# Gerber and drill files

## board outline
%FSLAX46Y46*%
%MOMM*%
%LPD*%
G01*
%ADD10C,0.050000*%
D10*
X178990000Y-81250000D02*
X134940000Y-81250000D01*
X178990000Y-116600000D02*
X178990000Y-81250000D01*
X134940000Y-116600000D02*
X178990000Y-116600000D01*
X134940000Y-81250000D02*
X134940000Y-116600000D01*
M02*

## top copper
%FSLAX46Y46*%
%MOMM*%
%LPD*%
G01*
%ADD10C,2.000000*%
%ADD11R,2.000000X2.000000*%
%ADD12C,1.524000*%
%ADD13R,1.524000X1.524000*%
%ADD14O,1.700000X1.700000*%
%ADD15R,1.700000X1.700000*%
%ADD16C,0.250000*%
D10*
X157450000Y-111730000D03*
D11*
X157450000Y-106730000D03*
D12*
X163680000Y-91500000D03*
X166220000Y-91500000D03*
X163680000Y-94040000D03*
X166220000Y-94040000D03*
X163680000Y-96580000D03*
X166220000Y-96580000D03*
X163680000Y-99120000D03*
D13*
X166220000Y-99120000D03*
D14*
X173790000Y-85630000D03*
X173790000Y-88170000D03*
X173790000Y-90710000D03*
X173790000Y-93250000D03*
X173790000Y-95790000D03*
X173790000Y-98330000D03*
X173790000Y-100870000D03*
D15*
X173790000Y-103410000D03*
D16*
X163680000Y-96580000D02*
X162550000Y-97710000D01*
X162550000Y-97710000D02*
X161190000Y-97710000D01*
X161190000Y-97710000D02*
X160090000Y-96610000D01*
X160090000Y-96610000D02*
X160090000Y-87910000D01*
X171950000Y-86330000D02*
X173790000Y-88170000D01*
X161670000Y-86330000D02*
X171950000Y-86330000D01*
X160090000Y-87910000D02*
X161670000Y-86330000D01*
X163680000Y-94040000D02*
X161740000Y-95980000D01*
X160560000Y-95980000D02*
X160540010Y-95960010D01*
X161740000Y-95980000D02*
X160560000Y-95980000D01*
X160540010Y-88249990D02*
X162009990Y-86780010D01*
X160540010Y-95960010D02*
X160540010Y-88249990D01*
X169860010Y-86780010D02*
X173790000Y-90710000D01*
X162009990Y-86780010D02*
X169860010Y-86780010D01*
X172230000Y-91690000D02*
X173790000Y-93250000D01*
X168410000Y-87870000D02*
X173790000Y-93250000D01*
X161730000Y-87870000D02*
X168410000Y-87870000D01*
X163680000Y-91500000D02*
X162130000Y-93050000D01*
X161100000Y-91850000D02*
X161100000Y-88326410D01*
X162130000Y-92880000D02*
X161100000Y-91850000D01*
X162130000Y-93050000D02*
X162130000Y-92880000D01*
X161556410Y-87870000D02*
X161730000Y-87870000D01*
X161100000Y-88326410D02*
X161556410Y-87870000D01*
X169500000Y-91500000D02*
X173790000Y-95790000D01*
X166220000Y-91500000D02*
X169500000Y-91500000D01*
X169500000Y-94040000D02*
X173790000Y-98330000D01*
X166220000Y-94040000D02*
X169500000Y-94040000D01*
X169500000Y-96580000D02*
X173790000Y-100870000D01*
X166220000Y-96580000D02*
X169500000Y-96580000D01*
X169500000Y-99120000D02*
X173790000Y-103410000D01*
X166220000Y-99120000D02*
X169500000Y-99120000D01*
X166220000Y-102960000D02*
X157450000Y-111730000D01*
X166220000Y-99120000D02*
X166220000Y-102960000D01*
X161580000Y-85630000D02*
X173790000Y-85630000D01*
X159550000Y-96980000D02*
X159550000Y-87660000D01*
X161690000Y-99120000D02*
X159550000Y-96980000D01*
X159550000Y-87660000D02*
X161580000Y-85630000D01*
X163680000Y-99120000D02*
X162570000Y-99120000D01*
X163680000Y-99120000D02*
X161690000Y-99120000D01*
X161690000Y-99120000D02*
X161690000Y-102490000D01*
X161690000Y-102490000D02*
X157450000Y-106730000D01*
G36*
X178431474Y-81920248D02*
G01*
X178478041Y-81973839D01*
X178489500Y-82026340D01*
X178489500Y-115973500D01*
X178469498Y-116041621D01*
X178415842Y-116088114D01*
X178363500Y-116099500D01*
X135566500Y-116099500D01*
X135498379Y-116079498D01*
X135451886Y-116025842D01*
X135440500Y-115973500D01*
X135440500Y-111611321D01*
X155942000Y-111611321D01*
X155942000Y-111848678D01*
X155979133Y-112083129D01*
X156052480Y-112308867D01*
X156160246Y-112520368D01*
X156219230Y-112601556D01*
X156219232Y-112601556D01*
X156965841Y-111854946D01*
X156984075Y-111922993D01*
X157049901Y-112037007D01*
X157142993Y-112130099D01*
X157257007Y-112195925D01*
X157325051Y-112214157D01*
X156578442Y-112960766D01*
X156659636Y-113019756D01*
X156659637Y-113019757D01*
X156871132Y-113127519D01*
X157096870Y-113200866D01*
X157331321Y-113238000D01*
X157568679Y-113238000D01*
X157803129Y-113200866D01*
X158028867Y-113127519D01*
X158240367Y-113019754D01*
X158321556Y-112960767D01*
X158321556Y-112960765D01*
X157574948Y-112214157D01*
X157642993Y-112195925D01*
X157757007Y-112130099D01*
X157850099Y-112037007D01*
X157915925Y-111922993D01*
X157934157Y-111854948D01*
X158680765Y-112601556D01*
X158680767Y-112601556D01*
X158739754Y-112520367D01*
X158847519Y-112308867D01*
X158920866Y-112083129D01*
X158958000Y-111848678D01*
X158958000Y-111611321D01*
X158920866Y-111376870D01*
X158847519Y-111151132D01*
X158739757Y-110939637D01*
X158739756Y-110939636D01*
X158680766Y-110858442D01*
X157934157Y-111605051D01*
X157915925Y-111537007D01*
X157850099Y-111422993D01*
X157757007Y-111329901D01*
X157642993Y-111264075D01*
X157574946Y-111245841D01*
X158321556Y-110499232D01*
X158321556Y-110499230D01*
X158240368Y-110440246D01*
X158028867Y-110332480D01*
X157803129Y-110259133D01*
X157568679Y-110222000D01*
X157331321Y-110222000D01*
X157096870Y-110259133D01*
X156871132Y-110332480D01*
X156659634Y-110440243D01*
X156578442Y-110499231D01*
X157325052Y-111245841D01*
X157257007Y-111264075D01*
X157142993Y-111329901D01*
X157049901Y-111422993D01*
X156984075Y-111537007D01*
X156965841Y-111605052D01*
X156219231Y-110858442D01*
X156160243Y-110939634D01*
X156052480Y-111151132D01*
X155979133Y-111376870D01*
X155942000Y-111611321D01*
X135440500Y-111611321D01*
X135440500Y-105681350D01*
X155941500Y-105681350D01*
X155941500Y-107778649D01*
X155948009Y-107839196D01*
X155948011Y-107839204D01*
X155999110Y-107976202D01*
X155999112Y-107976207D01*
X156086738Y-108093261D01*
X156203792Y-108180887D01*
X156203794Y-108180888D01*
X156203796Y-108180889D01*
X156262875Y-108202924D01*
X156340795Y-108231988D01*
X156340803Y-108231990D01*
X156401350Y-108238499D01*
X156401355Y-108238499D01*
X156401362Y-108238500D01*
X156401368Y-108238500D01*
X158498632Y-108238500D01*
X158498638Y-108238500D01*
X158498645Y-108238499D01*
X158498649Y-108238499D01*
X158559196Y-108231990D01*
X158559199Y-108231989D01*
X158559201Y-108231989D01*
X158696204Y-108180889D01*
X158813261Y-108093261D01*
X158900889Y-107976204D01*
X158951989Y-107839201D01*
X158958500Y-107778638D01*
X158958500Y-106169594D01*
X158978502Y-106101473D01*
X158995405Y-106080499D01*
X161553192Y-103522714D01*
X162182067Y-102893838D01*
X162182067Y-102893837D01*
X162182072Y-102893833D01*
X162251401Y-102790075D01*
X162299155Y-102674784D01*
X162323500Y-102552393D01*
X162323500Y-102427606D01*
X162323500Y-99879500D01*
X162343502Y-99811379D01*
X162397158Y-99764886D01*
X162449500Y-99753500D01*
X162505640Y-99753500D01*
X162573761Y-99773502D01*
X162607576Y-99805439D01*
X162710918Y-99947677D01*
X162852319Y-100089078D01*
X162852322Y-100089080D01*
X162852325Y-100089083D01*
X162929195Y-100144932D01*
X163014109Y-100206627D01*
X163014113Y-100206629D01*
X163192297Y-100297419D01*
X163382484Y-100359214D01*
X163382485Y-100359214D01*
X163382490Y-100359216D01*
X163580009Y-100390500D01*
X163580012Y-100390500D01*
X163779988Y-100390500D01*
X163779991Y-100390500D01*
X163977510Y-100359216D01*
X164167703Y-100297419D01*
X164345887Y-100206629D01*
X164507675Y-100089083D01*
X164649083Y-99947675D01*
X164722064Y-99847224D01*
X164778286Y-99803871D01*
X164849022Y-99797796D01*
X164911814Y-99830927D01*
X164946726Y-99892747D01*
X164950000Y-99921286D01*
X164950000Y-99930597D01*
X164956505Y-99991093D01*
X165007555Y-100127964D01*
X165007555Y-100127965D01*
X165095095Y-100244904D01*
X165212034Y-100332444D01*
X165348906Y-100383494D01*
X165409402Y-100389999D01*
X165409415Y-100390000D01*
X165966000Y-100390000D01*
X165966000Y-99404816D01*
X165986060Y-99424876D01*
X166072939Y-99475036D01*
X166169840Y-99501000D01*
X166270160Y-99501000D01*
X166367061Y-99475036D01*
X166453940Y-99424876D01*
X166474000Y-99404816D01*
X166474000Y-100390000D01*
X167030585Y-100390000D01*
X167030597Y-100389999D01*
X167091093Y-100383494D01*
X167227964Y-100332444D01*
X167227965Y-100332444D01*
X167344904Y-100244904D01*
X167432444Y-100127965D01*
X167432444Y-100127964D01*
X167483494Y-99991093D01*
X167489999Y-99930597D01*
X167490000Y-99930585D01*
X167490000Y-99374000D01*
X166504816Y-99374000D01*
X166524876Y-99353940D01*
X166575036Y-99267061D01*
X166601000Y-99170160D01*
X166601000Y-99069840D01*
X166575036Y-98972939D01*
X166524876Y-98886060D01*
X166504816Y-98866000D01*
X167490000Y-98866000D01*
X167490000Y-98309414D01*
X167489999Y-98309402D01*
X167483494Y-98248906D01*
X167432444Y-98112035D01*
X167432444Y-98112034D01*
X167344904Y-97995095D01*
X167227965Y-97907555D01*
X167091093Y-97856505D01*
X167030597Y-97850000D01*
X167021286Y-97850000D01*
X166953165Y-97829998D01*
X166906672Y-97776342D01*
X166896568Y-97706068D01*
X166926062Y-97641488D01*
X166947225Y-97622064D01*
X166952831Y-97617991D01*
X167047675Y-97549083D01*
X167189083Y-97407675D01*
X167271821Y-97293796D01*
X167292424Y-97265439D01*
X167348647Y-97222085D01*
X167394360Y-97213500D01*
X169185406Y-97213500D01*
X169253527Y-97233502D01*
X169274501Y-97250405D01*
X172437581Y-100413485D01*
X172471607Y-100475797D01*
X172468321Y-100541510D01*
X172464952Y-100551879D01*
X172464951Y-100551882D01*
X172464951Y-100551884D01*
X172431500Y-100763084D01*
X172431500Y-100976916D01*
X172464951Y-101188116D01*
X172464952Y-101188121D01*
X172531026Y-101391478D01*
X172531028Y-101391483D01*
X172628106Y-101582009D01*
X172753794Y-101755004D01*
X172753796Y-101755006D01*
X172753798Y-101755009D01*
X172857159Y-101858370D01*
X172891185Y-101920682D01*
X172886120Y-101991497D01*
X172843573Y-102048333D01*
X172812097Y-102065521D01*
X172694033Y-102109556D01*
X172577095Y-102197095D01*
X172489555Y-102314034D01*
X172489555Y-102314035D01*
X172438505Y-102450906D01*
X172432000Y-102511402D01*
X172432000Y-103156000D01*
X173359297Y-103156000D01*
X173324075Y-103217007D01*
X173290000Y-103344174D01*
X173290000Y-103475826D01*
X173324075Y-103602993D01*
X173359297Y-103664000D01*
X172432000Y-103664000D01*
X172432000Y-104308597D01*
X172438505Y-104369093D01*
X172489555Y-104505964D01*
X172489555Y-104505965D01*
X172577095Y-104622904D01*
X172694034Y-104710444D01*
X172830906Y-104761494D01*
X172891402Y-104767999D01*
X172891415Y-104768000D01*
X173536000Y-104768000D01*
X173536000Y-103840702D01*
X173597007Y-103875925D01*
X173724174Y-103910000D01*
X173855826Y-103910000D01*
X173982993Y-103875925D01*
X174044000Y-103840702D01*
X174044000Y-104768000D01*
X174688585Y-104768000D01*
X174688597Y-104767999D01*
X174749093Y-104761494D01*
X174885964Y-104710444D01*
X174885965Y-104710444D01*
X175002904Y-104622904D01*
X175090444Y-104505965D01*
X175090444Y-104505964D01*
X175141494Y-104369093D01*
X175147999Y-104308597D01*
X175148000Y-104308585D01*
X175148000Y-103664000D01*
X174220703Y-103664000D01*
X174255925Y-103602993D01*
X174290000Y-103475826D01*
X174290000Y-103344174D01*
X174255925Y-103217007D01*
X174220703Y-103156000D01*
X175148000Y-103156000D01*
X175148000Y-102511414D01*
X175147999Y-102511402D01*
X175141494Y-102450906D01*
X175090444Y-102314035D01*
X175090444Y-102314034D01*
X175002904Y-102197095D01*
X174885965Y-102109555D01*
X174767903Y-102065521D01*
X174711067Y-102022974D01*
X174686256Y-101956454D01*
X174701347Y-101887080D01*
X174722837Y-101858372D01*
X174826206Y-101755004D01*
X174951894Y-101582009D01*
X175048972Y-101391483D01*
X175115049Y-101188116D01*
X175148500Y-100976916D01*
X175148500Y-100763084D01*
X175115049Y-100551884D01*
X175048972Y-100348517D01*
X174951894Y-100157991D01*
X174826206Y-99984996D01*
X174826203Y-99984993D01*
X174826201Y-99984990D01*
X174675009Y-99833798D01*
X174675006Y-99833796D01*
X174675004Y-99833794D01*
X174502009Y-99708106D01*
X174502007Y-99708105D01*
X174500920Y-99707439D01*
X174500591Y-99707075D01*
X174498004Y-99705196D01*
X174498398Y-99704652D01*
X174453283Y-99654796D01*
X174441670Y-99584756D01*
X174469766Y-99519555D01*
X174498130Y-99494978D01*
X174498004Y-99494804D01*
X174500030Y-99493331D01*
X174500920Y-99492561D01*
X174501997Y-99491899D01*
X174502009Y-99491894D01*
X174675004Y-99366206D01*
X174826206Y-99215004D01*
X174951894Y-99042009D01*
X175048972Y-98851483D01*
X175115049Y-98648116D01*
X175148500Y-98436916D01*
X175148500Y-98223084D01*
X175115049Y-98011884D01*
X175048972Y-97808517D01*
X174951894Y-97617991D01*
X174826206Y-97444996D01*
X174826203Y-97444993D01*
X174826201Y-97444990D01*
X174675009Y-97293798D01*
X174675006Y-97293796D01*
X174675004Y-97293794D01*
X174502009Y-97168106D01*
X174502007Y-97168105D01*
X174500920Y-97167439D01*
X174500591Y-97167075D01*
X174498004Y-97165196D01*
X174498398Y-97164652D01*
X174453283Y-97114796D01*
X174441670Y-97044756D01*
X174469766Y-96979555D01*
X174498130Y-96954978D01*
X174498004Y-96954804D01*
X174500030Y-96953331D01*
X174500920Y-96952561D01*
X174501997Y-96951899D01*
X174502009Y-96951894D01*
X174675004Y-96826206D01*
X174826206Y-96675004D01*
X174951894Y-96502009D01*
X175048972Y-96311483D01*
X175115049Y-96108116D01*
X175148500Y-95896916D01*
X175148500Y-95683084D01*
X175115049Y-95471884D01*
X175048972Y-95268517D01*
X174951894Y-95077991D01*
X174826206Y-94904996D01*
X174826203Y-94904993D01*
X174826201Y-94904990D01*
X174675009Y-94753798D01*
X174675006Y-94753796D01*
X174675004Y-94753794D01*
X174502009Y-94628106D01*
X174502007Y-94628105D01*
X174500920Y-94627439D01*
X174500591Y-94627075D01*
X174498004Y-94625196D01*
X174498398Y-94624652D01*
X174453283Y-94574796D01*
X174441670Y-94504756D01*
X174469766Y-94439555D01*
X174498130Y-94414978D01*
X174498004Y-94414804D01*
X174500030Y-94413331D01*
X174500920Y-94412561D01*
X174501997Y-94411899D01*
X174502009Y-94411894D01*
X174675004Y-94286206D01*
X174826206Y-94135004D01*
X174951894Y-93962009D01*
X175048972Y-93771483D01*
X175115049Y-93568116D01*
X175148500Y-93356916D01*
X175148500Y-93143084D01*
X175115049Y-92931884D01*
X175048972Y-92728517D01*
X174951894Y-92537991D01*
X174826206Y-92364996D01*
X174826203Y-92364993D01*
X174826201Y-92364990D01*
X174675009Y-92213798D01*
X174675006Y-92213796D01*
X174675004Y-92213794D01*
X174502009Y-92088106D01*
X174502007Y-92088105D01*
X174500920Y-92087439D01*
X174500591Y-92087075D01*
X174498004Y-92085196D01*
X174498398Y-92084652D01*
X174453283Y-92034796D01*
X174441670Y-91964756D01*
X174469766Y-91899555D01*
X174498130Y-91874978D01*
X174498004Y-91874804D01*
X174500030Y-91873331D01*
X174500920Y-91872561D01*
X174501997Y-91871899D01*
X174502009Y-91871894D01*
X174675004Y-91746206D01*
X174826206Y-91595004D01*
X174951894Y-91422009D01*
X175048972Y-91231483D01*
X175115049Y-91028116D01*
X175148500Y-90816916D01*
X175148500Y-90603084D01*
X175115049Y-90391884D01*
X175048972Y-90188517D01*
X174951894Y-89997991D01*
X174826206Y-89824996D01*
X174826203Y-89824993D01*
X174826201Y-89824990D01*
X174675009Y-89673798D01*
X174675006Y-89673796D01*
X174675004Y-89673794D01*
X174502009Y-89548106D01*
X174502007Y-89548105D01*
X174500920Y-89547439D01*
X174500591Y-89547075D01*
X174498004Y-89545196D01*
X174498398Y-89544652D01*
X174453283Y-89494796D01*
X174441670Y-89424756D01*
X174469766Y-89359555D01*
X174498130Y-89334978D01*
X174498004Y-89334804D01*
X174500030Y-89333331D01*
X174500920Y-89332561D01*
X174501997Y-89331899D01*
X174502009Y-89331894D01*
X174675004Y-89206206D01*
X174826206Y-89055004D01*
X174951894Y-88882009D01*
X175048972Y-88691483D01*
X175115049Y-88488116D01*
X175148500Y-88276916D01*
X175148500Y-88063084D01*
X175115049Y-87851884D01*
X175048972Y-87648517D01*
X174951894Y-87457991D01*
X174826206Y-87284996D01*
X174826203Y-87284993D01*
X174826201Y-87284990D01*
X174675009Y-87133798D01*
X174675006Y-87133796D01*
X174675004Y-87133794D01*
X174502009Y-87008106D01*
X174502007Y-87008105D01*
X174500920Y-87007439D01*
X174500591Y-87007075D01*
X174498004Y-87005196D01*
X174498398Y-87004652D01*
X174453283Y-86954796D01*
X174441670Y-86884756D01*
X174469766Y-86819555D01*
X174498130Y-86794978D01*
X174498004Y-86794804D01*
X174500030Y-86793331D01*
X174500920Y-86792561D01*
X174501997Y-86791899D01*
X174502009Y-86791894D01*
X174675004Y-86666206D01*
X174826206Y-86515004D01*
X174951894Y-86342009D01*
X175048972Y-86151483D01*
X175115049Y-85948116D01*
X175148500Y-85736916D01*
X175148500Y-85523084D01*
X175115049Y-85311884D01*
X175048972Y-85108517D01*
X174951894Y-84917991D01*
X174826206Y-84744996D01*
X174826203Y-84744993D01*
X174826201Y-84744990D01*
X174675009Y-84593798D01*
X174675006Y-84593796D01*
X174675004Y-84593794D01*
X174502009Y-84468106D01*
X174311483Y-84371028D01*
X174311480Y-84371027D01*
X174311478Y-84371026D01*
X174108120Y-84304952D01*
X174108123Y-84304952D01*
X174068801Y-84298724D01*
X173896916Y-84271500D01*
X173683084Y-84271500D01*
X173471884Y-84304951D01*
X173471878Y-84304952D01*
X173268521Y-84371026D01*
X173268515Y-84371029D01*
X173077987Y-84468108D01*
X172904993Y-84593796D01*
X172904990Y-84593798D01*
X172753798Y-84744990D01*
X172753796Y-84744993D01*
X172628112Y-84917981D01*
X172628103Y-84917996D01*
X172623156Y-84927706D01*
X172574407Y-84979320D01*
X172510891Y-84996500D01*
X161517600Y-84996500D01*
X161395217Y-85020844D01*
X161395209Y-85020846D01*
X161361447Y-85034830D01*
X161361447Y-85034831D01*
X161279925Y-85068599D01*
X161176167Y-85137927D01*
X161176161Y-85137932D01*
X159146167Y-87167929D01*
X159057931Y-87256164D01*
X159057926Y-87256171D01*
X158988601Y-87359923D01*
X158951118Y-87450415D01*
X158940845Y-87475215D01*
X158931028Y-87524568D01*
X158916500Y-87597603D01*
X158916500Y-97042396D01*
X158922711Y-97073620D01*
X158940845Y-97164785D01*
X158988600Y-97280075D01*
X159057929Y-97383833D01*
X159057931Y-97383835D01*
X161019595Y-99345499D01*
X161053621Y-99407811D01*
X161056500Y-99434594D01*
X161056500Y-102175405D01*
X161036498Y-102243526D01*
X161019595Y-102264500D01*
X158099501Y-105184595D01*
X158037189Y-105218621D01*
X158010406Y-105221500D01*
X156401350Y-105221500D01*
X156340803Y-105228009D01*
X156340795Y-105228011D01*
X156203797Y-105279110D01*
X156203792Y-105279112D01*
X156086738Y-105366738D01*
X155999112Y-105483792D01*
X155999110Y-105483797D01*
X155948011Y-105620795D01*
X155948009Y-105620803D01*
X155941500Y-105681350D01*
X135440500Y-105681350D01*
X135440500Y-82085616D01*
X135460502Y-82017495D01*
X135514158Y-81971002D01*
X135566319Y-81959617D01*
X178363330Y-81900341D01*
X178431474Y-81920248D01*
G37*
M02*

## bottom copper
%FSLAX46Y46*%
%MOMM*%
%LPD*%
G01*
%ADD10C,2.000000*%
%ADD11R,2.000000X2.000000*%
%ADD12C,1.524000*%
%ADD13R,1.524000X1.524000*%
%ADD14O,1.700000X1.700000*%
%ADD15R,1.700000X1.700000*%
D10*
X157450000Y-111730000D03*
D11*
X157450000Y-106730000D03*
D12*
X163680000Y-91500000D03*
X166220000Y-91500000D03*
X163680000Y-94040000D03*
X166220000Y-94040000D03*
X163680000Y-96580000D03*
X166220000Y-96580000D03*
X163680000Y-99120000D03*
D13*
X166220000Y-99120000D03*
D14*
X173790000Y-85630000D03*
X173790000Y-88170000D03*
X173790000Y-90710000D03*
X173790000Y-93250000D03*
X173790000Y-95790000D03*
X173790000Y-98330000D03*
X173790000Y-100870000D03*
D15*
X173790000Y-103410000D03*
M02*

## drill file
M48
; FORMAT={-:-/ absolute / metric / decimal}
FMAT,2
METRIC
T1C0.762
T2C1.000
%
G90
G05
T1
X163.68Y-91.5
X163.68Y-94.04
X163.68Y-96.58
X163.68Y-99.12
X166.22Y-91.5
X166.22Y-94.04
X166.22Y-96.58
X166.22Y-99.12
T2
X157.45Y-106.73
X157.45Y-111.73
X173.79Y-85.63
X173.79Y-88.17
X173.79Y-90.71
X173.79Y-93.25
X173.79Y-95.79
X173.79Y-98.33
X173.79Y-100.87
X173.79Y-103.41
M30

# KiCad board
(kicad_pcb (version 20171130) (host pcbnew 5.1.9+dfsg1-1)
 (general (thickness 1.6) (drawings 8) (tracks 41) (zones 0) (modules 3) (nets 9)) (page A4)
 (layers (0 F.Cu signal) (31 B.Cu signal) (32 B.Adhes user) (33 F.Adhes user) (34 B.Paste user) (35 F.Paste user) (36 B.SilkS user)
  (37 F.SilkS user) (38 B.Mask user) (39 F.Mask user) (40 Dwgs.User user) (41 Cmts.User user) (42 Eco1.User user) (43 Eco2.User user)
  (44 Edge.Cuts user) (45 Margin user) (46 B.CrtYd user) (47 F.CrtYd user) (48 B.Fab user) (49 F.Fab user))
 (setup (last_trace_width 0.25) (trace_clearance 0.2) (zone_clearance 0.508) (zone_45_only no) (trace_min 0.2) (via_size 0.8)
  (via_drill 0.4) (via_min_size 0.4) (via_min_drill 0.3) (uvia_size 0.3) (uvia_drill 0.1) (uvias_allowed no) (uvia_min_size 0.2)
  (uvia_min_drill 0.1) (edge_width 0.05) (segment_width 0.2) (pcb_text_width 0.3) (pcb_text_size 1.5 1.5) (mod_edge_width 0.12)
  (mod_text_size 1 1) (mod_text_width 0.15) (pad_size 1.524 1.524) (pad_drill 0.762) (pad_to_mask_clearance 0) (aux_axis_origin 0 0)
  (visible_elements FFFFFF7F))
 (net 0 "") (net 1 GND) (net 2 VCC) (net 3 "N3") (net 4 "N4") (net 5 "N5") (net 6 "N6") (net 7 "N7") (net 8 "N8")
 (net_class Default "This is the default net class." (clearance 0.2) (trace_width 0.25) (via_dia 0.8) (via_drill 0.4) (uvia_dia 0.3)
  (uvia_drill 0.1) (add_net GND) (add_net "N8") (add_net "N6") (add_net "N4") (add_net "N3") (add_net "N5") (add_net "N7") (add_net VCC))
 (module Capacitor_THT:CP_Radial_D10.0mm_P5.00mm (layer F.Cu) (at 157.45 106.73 270)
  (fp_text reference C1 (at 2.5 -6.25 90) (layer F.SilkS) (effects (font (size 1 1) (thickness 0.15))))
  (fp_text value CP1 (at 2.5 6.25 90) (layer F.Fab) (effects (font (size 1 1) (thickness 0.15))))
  (pad 2 thru_hole circle (at 5 0 270) (size 2 2) (drill 1) (layers *.Cu *.Mask) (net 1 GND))
  (pad 1 thru_hole rect (at 0 0 270) (size 2 2) (drill 1) (layers *.Cu *.Mask) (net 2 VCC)))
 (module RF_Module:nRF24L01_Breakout (layer F.Cu) (at 166.22 99.12 180)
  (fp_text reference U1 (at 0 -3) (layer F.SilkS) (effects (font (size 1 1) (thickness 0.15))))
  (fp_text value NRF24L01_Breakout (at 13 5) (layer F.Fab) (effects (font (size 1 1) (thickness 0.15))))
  (pad 8 thru_hole circle (at 2.54 7.62 180) (size 1.524 1.524) (drill 0.762) (layers *.Cu *.Mask) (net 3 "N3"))
  (pad 7 thru_hole circle (at 0 7.62 180) (size 1.524 1.524) (drill 0.762) (layers *.Cu *.Mask) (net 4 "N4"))
  (pad 6 thru_hole circle (at 2.54 5.08 180) (size 1.524 1.524) (drill 0.762) (layers *.Cu *.Mask) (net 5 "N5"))
  (pad 5 thru_hole circle (at 0 5.08 180) (size 1.524 1.524) (drill 0.762) (layers *.Cu *.Mask) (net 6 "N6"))
  (pad 4 thru_hole circle (at 2.54 2.54 180) (size 1.524 1.524) (drill 0.762) (layers *.Cu *.Mask) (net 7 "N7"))
  (pad 3 thru_hole circle (at 0 2.54 180) (size 1.524 1.524) (drill 0.762) (layers *.Cu *.Mask) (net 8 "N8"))
  (pad 2 thru_hole circle (at 2.54 0 180) (size 1.524 1.524) (drill 0.762) (layers *.Cu *.Mask) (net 2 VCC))
  (pad 1 thru_hole rect (at 0 0 180) (size 1.524 1.524) (drill 0.762) (layers *.Cu *.Mask) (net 1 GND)))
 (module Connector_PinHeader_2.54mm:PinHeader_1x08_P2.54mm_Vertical (layer F.Cu) (at 173.79 103.41 180)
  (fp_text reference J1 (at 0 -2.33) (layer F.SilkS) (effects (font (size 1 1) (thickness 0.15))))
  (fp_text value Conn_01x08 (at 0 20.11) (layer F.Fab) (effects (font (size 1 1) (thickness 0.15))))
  (pad 8 thru_hole oval (at 0 17.78 180) (size 1.7 1.7) (drill 1) (layers *.Cu *.Mask) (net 2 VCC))
  (pad 7 thru_hole oval (at 0 15.24 180) (size 1.7 1.7) (drill 1) (layers *.Cu *.Mask) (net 7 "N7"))
  (pad 6 thru_hole oval (at 0 12.7 180) (size 1.7 1.7) (drill 1) (layers *.Cu *.Mask) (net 5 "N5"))
  (pad 5 thru_hole oval (at 0 10.16 180) (size 1.7 1.7) (drill 1) (layers *.Cu *.Mask) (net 3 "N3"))
  (pad 4 thru_hole oval (at 0 7.62 180) (size 1.7 1.7) (drill 1) (layers *.Cu *.Mask) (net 4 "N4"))
  (pad 3 thru_hole oval (at 0 5.08 180) (size 1.7 1.7) (drill 1) (layers *.Cu *.Mask) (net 6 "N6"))
  (pad 2 thru_hole oval (at 0 2.54 180) (size 1.7 1.7) (drill 1) (layers *.Cu *.Mask) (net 8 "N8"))
  (pad 1 thru_hole rect (at 0 0 180) (size 1.7 1.7) (drill 1) (layers *.Cu *.Mask) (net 1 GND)))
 (gr_line (start 178.99 81.25) (end 134.94 81.25) (layer Edge.Cuts) (width 0.05))
 (gr_line (start 178.99 116.6) (end 178.99 81.25) (layer Edge.Cuts) (width 0.05))
 (gr_line (start 134.94 116.6) (end 178.99 116.6) (layer Edge.Cuts) (width 0.05))
 (gr_line (start 134.94 81.25) (end 134.94 116.6) (layer Edge.Cuts) (width 0.05))
 (segment (start 163.68 96.58) (end 162.55 97.71) (width 0.25) (layer F.Cu) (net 7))
 (segment (start 162.55 97.71) (end 161.19 97.71) (width 0.25) (layer F.Cu) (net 7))
 (segment (start 161.19 97.71) (end 160.09 96.61) (width 0.25) (layer F.Cu) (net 7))
 (segment (start 160.09 96.61) (end 160.09 87.91) (width 0.25) (layer F.Cu) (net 7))
 (segment (start 171.95 86.33) (end 173.79 88.17) (width 0.25) (layer F.Cu) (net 7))
 (segment (start 161.67 86.33) (end 171.95 86.33) (width 0.25) (layer F.Cu) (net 7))
 (segment (start 160.09 87.91) (end 161.67 86.33) (width 0.25) (layer F.Cu) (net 7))
 (segment (start 163.68 94.04) (end 161.74 95.98) (width 0.25) (layer F.Cu) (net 5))
 (segment (start 160.56 95.98) (end 160.54001 95.96001) (width 0.25) (layer F.Cu) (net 5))
 (segment (start 161.74 95.98) (end 160.56 95.98) (width 0.25) (layer F.Cu) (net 5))
 (segment (start 160.54001 88.24999) (end 162.00999 86.78001) (width 0.25) (layer F.Cu) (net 5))
 (segment (start 160.54001 95.96001) (end 160.54001 88.24999) (width 0.25) (layer F.Cu) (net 5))
 (segment (start 169.86001 86.78001) (end 173.79 90.71) (width 0.25) (layer F.Cu) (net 5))
 (segment (start 162.00999 86.78001) (end 169.86001 86.78001) (width 0.25) (layer F.Cu) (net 5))
 (segment (start 172.23 91.69) (end 173.79 93.25) (width 0.25) (layer F.Cu) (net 3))
 (segment (start 168.41 87.87) (end 173.79 93.25) (width 0.25) (layer F.Cu) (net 3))
 (segment (start 161.73 87.87) (end 168.41 87.87) (width 0.25) (layer F.Cu) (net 3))
 (segment (start 163.68 91.5) (end 162.13 93.05) (width 0.25) (layer F.Cu) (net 3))
 (segment (start 161.1 91.85) (end 161.1 88.32641) (width 0.25) (layer F.Cu) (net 3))
 (segment (start 162.13 92.88) (end 161.1 91.85) (width 0.25) (layer F.Cu) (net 3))
 (segment (start 162.13 93.05) (end 162.13 92.88) (width 0.25) (layer F.Cu) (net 3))
 (segment (start 161.55641 87.87) (end 161.73 87.87) (width 0.25) (layer F.Cu) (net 3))
 (segment (start 161.1 88.32641) (end 161.55641 87.87) (width 0.25) (layer F.Cu) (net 3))
 (segment (start 169.5 91.5) (end 173.79 95.79) (width 0.25) (layer F.Cu) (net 4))
 (segment (start 166.22 91.5) (end 169.5 91.5) (width 0.25) (layer F.Cu) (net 4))
 (segment (start 169.5 94.04) (end 173.79 98.33) (width 0.25) (layer F.Cu) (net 6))
 (segment (start 166.22 94.04) (end 169.5 94.04) (width 0.25) (layer F.Cu) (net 6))
 (segment (start 169.5 96.58) (end 173.79 100.87) (width 0.25) (layer F.Cu) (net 8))
 (segment (start 166.22 96.58) (end 169.5 96.58) (width 0.25) (layer F.Cu) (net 8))
 (segment (start 169.5 99.12) (end 173.79 103.41) (width 0.25) (layer F.Cu) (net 1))
 (segment (start 166.22 99.12) (end 169.5 99.12) (width 0.25) (layer F.Cu) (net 1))
 (segment (start 166.22 102.96) (end 157.45 111.73) (width 0.25) (layer F.Cu) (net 1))
 (segment (start 166.22 99.12) (end 166.22 102.96) (width 0.25) (layer F.Cu) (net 1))
 (segment (start 161.58 85.63) (end 173.79 85.63) (width 0.25) (layer F.Cu) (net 2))
 (segment (start 159.55 96.98) (end 159.55 87.66) (width 0.25) (layer F.Cu) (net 2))
 (segment (start 161.69 99.12) (end 159.55 96.98) (width 0.25) (layer F.Cu) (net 2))
 (segment (start 159.55 87.66) (end 161.58 85.63) (width 0.25) (layer F.Cu) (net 2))
 (segment (start 163.68 99.12) (end 162.57 99.12) (width 0.25) (layer F.Cu) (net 2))
 (segment (start 163.68 99.12) (end 161.69 99.12) (width 0.25) (layer F.Cu) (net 2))
 (segment (start 161.69 99.12) (end 161.69 102.49) (width 0.25) (layer F.Cu) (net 2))
 (segment (start 161.69 102.49) (end 157.45 106.73) (width 0.25) (layer F.Cu) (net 2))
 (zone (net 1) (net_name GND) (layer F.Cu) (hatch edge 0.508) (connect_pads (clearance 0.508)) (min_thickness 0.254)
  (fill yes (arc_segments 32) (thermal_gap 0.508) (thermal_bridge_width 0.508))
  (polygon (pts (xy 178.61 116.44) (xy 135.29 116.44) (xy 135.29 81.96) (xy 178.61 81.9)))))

